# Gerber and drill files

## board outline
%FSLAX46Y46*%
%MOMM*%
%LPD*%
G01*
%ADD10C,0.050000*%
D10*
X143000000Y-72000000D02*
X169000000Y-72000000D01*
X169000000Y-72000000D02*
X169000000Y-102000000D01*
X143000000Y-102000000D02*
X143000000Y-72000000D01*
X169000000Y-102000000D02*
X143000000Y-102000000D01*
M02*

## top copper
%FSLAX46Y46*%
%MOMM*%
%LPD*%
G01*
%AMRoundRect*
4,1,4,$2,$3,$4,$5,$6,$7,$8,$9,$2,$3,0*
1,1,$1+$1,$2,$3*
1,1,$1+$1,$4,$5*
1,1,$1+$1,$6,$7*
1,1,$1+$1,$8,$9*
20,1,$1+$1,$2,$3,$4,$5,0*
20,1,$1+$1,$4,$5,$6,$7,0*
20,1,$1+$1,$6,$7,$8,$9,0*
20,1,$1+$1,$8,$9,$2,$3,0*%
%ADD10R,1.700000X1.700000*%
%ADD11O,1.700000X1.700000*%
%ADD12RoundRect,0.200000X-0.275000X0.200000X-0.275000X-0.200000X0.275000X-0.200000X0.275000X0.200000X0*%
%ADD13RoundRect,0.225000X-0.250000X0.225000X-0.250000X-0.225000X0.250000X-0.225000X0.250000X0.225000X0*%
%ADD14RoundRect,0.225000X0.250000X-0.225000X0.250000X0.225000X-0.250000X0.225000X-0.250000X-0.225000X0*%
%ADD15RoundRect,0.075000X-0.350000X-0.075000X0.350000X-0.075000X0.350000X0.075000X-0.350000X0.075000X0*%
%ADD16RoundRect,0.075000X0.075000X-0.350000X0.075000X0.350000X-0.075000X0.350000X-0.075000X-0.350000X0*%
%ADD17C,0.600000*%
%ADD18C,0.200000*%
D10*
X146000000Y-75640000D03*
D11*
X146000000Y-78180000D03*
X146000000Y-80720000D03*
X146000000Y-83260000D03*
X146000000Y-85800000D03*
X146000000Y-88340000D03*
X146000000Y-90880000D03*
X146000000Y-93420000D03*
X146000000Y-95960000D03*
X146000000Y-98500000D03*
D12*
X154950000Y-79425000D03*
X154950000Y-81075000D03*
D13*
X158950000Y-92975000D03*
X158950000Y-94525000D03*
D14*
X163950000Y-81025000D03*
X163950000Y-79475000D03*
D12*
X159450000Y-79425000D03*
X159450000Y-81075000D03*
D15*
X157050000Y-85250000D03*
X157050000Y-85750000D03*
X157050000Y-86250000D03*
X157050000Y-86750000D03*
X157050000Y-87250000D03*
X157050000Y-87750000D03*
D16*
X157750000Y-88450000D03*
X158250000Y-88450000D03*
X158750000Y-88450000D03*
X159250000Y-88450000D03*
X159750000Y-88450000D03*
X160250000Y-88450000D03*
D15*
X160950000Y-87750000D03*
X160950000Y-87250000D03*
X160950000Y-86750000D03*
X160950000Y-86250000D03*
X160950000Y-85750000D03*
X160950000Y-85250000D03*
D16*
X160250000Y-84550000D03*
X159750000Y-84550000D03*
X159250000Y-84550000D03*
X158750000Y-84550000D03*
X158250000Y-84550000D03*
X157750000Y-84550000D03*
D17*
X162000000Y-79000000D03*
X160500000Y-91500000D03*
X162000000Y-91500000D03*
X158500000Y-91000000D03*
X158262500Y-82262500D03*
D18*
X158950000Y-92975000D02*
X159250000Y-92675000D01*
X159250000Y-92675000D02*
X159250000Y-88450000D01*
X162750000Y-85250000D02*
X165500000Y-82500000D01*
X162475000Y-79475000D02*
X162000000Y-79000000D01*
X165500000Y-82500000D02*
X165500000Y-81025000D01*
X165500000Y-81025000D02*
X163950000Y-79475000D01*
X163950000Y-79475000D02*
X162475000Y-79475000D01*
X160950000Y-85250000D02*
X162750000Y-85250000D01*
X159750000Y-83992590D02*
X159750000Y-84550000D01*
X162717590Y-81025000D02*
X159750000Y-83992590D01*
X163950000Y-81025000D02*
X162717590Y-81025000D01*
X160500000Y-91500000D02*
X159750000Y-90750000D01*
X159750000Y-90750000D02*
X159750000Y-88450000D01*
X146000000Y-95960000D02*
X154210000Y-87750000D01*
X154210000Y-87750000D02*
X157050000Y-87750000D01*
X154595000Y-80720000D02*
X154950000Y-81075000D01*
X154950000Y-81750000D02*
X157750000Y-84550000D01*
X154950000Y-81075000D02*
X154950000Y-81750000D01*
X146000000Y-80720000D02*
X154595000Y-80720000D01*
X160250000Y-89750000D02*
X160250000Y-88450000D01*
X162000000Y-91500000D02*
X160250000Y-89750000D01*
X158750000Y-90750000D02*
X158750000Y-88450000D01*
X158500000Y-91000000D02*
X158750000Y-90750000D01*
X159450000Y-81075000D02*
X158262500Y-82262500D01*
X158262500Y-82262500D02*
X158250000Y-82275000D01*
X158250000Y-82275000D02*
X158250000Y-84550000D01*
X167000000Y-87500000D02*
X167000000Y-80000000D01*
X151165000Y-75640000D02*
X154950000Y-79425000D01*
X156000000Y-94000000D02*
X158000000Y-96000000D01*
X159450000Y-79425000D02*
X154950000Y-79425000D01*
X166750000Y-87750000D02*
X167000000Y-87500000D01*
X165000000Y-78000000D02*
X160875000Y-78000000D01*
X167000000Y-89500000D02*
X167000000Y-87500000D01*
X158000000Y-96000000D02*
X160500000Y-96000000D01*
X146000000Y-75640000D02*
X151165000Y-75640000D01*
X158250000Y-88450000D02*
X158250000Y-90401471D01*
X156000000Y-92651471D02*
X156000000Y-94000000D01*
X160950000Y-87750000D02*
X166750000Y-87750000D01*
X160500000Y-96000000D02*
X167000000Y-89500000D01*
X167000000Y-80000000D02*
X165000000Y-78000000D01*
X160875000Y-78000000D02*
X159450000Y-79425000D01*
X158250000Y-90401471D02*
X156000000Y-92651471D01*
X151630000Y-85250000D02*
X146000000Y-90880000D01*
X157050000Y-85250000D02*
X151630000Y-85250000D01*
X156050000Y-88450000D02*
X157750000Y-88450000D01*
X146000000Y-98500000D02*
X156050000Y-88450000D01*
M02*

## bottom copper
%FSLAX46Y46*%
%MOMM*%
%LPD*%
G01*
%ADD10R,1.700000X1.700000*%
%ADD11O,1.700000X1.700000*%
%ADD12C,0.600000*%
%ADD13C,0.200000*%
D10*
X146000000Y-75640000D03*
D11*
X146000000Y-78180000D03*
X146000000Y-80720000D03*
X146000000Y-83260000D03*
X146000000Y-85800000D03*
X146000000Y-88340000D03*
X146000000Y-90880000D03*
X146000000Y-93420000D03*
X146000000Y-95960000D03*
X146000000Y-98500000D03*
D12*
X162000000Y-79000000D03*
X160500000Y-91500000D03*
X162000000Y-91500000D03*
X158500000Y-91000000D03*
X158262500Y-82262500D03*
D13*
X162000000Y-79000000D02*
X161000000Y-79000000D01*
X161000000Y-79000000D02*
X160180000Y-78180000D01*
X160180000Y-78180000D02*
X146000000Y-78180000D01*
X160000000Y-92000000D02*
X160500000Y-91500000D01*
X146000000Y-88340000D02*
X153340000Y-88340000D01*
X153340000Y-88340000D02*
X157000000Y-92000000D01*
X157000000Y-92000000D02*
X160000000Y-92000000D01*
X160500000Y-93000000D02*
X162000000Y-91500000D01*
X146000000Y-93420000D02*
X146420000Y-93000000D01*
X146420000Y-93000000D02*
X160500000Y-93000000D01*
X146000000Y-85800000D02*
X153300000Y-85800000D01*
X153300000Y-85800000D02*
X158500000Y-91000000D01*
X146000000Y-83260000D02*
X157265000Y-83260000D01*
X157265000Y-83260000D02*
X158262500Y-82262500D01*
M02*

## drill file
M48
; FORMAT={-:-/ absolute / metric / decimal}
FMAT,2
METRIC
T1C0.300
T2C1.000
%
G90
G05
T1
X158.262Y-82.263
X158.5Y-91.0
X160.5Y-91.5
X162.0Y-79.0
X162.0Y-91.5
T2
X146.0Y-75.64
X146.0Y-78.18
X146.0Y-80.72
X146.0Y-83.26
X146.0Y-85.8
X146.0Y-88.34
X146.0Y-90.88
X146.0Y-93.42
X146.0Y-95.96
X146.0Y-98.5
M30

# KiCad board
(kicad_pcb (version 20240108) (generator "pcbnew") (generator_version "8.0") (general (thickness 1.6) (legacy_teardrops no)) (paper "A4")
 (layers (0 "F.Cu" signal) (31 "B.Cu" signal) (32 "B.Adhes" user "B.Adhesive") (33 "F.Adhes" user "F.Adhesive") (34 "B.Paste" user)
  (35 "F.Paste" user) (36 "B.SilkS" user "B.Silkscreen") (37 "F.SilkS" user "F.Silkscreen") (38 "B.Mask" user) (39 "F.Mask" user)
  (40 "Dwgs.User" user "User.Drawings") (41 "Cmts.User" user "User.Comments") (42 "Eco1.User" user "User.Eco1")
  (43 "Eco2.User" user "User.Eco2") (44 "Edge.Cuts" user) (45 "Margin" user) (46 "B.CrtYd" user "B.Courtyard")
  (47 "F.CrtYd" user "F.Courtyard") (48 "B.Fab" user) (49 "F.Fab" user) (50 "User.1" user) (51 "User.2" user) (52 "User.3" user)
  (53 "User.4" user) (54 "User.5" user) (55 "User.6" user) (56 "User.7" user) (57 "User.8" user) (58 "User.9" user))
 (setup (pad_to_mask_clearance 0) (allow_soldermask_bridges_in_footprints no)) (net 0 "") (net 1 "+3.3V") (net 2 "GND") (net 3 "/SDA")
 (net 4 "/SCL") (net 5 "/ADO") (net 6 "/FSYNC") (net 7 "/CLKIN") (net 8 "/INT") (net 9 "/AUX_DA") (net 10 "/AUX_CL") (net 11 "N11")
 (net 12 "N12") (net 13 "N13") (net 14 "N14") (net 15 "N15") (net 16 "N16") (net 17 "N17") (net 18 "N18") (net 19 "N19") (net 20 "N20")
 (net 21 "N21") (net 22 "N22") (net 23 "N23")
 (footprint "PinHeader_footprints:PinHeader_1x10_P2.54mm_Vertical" (layer "F.Cu") (at 146 75.64)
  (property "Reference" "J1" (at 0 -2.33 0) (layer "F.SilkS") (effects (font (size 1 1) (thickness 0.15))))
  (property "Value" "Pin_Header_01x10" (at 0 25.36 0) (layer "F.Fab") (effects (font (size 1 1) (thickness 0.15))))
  (pad "1" thru_hole rect (at 0 0) (size 1.7 1.7) (drill 1) (layers "*.Cu" "*.Mask") (remove_unused_layers no) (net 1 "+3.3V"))
  (pad "2" thru_hole oval (at 0 2.54) (size 1.7 1.7) (drill 1) (layers "*.Cu" "*.Mask") (remove_unused_layers no) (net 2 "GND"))
  (pad "3" thru_hole oval (at 0 5.08) (size 1.7 1.7) (drill 1) (layers "*.Cu" "*.Mask") (remove_unused_layers no) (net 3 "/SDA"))
  (pad "4" thru_hole oval (at 0 7.62) (size 1.7 1.7) (drill 1) (layers "*.Cu" "*.Mask") (remove_unused_layers no) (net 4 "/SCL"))
  (pad "5" thru_hole oval (at 0 10.16) (size 1.7 1.7) (drill 1) (layers "*.Cu" "*.Mask") (remove_unused_layers no) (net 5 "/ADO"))
  (pad "6" thru_hole oval (at 0 12.7) (size 1.7 1.7) (drill 1) (layers "*.Cu" "*.Mask") (remove_unused_layers no) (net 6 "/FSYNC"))
  (pad "7" thru_hole oval (at 0 15.24) (size 1.7 1.7) (drill 1) (layers "*.Cu" "*.Mask") (remove_unused_layers no) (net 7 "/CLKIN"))
  (pad "8" thru_hole oval (at 0 17.78) (size 1.7 1.7) (drill 1) (layers "*.Cu" "*.Mask") (remove_unused_layers no) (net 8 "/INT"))
  (pad "9" thru_hole oval (at 0 20.32) (size 1.7 1.7) (drill 1) (layers "*.Cu" "*.Mask") (remove_unused_layers no) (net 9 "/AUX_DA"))
  (pad "10" thru_hole oval (at 0 22.86) (size 1.7 1.7) (drill 1) (layers "*.Cu" "*.Mask") (remove_unused_layers no) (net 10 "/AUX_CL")))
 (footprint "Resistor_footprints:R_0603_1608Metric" (layer "F.Cu") (at 154.95 80.25 -90)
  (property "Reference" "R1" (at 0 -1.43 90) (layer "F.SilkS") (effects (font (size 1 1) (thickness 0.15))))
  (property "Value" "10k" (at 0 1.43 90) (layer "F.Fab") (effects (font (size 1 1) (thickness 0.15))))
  (pad "1" smd roundrect (at -0.825 0 270) (size 0.8 0.95) (layers "F.Cu" "F.Paste" "F.Mask") (roundrect_rratio 0.25) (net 1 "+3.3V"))
  (pad "2" smd roundrect (at 0.825 0 270) (size 0.8 0.95) (layers "F.Cu" "F.Paste" "F.Mask") (roundrect_rratio 0.25) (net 3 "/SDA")))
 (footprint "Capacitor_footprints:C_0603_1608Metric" (layer "F.Cu") (at 158.95 93.75 -90)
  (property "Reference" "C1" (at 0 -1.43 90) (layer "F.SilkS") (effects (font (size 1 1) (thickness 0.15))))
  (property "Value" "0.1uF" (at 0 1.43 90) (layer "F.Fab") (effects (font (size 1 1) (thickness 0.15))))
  (pad "1" smd roundrect (at -0.775 0 270) (size 0.9 0.95) (layers "F.Cu" "F.Paste" "F.Mask") (roundrect_rratio 0.25) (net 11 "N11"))
  (pad "2" smd roundrect (at 0.775 0 270) (size 0.9 0.95) (layers "F.Cu" "F.Paste" "F.Mask") (roundrect_rratio 0.25) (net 2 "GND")))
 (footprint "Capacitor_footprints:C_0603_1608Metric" (layer "F.Cu") (at 163.95 80.25 90)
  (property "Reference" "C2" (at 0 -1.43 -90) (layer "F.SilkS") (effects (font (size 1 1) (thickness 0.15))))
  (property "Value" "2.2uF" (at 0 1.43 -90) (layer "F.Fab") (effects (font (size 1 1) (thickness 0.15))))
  (pad "1" smd roundrect (at -0.775 0 90) (size 0.9 0.95) (layers "F.Cu" "F.Paste" "F.Mask") (roundrect_rratio 0.25) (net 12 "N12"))
  (pad "2" smd roundrect (at 0.775 0 90) (size 0.9 0.95) (layers "F.Cu" "F.Paste" "F.Mask") (roundrect_rratio 0.25) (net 2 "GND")))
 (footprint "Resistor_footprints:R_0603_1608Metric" (layer "F.Cu") (at 159.45 80.25 -90)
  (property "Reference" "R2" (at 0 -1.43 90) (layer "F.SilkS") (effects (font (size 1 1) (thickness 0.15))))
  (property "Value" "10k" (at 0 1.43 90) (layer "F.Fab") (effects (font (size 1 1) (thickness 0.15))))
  (pad "1" smd roundrect (at -0.825 0 270) (size 0.8 0.95) (layers "F.Cu" "F.Paste" "F.Mask") (roundrect_rratio 0.25) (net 1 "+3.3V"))
  (pad "2" smd roundrect (at 0.825 0 270) (size 0.8 0.95) (layers "F.Cu" "F.Paste" "F.Mask") (roundrect_rratio 0.25) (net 4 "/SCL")))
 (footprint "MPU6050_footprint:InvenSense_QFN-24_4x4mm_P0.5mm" (layer "F.Cu") (at 159 86.5)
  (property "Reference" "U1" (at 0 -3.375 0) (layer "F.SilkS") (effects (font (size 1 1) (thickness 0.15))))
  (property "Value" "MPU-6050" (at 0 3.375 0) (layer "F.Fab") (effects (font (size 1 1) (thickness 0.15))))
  (pad "1" smd roundrect (at -1.95 -1.25) (size 0.85 0.3) (layers "F.Cu" "F.Paste" "F.Mask") (roundrect_rratio 0.25) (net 7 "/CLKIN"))
  (pad "2" smd roundrect (at -1.95 -0.75) (size 0.85 0.3) (layers "F.Cu" "F.Paste" "F.Mask") (roundrect_rratio 0.25) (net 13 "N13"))
  (pad "3" smd roundrect (at -1.95 -0.25) (size 0.85 0.3) (layers "F.Cu" "F.Paste" "F.Mask") (roundrect_rratio 0.25) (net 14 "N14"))
  (pad "4" smd roundrect (at -1.95 0.25) (size 0.85 0.3) (layers "F.Cu" "F.Paste" "F.Mask") (roundrect_rratio 0.25) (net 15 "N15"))
  (pad "5" smd roundrect (at -1.95 0.75) (size 0.85 0.3) (layers "F.Cu" "F.Paste" "F.Mask") (roundrect_rratio 0.25) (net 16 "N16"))
  (pad "6" smd roundrect (at -1.95 1.25) (size 0.85 0.3) (layers "F.Cu" "F.Paste" "F.Mask") (roundrect_rratio 0.25) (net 9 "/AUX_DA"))
  (pad "7" smd roundrect (at -1.25 1.95 90) (size 0.85 0.3) (layers "F.Cu" "F.Paste" "F.Mask") (roundrect_rratio 0.25) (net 10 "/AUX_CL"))
  (pad "8" smd roundrect (at -0.75 1.95 90) (size 0.85 0.3) (layers "F.Cu" "F.Paste" "F.Mask") (roundrect_rratio 0.25) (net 1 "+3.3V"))
  (pad "9" smd roundrect (at -0.25 1.95 90) (size 0.85 0.3) (layers "F.Cu" "F.Paste" "F.Mask") (roundrect_rratio 0.25) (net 5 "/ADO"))
  (pad "10" smd roundrect (at 0.25 1.95 90) (size 0.85 0.3) (layers "F.Cu" "F.Paste" "F.Mask") (roundrect_rratio 0.25) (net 11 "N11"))
  (pad "11" smd roundrect (at 0.75 1.95 90) (size 0.85 0.3) (layers "F.Cu" "F.Paste" "F.Mask") (roundrect_rratio 0.25) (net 6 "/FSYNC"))
  (pad "12" smd roundrect (at 1.25 1.95 90) (size 0.85 0.3) (layers "F.Cu" "F.Paste" "F.Mask") (roundrect_rratio 0.25) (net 8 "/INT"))
  (pad "13" smd roundrect (at 1.95 1.25) (size 0.85 0.3) (layers "F.Cu" "F.Paste" "F.Mask") (roundrect_rratio 0.25) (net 1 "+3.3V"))
  (pad "14" smd roundrect (at 1.95 0.75) (size 0.85 0.3) (layers "F.Cu" "F.Paste" "F.Mask") (roundrect_rratio 0.25) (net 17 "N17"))
  (pad "15" smd roundrect (at 1.95 0.25) (size 0.85 0.3) (layers "F.Cu" "F.Paste" "F.Mask") (roundrect_rratio 0.25) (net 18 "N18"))
  (pad "16" smd roundrect (at 1.95 -0.25) (size 0.85 0.3) (layers "F.Cu" "F.Paste" "F.Mask") (roundrect_rratio 0.25) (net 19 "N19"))
  (pad "17" smd roundrect (at 1.95 -0.75) (size 0.85 0.3) (layers "F.Cu" "F.Paste" "F.Mask") (roundrect_rratio 0.25) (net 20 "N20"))
  (pad "18" smd roundrect (at 1.95 -1.25) (size 0.85 0.3) (layers "F.Cu" "F.Paste" "F.Mask") (roundrect_rratio 0.25) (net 2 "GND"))
  (pad "19" smd roundrect (at 1.25 -1.95 90) (size 0.85 0.3) (layers "F.Cu" "F.Paste" "F.Mask") (roundrect_rratio 0.25) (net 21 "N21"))
  (pad "20" smd roundrect (at 0.75 -1.95 90) (size 0.85 0.3) (layers "F.Cu" "F.Paste" "F.Mask") (roundrect_rratio 0.25) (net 12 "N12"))
  (pad "21" smd roundrect (at 0.25 -1.95 90) (size 0.85 0.3) (layers "F.Cu" "F.Paste" "F.Mask") (roundrect_rratio 0.25) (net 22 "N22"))
  (pad "22" smd roundrect (at -0.25 -1.95 90) (size 0.85 0.3) (layers "F.Cu" "F.Paste" "F.Mask") (roundrect_rratio 0.25) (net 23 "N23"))
  (pad "23" smd roundrect (at -0.75 -1.95 90) (size 0.85 0.3) (layers "F.Cu" "F.Paste" "F.Mask") (roundrect_rratio 0.25) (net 4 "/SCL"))
  (pad "24" smd roundrect (at -1.25 -1.95 90) (size 0.85 0.3) (layers "F.Cu" "F.Paste" "F.Mask") (roundrect_rratio 0.25) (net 3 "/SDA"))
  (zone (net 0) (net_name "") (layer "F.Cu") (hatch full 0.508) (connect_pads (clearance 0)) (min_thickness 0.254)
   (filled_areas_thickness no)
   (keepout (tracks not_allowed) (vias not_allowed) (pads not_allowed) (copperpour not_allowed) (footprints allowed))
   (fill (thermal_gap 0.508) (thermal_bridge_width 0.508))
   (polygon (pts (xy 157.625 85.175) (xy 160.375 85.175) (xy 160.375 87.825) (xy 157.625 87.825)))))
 (gr_line (start 143 72) (end 169 72) (stroke (width 0.05) (type default)) (layer "Edge.Cuts"))
 (gr_line (start 169 72) (end 169 102) (stroke (width 0.05) (type default)) (layer "Edge.Cuts"))
 (gr_line (start 143 102) (end 143 72) (stroke (width 0.05) (type default)) (layer "Edge.Cuts"))
 (gr_line (start 169 102) (end 143 102) (stroke (width 0.05) (type default)) (layer "Edge.Cuts"))
 (segment (start 158.95 92.975) (end 159.25 92.675) (width 0.2) (layer "F.Cu") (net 11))
 (segment (start 159.25 92.675) (end 159.25 88.45) (width 0.2) (layer "F.Cu") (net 11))
 (segment (start 162.75 85.25) (end 165.5 82.5) (width 0.2) (layer "F.Cu") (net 2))
 (segment (start 162.475 79.475) (end 162 79) (width 0.2) (layer "F.Cu") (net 2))
 (segment (start 165.5 82.5) (end 165.5 81.025) (width 0.2) (layer "F.Cu") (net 2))
 (segment (start 165.5 81.025) (end 163.95 79.475) (width 0.2) (layer "F.Cu") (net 2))
 (segment (start 163.95 79.475) (end 162.475 79.475) (width 0.2) (layer "F.Cu") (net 2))
 (segment (start 160.95 85.25) (end 162.75 85.25) (width 0.2) (layer "F.Cu") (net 2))
 (via (at 162 79) (size 0.6) (drill 0.3) (layers "F.Cu" "B.Cu") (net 2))
 (segment (start 162 79) (end 161 79) (width 0.2) (layer "B.Cu") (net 2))
 (segment (start 161 79) (end 160.18 78.18) (width 0.2) (layer "B.Cu") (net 2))
 (segment (start 160.18 78.18) (end 146 78.18) (width 0.2) (layer "B.Cu") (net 2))
 (segment (start 159.75 83.99259) (end 159.75 84.55) (width 0.2) (layer "F.Cu") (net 12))
 (segment (start 162.71759 81.025) (end 159.75 83.99259) (width 0.2) (layer "F.Cu") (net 12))
 (segment (start 163.95 81.025) (end 162.71759 81.025) (width 0.2) (layer "F.Cu") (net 12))
 (segment (start 160.5 91.5) (end 159.75 90.75) (width 0.2) (layer "F.Cu") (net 6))
 (segment (start 159.75 90.75) (end 159.75 88.45) (width 0.2) (layer "F.Cu") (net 6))
 (via (at 160.5 91.5) (size 0.6) (drill 0.3) (layers "F.Cu" "B.Cu") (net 6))
 (segment (start 160 92) (end 160.5 91.5) (width 0.2) (layer "B.Cu") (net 6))
 (segment (start 146 88.34) (end 153.34 88.34) (width 0.2) (layer "B.Cu") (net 6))
 (segment (start 153.34 88.34) (end 157 92) (width 0.2) (layer "B.Cu") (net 6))
 (segment (start 157 92) (end 160 92) (width 0.2) (layer "B.Cu") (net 6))
 (segment (start 146 95.96) (end 154.21 87.75) (width 0.2) (layer "F.Cu") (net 9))
 (segment (start 154.21 87.75) (end 157.05 87.75) (width 0.2) (layer "F.Cu") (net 9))
 (segment (start 154.595 80.72) (end 154.95 81.075) (width 0.2) (layer "F.Cu") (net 3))
 (segment (start 154.95 81.75) (end 157.75 84.55) (width 0.2) (layer "F.Cu") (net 3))
 (segment (start 154.95 81.075) (end 154.95 81.75) (width 0.2) (layer "F.Cu") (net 3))
 (segment (start 146 80.72) (end 154.595 80.72) (width 0.2) (layer "F.Cu") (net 3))
 (segment (start 160.25 89.75) (end 160.25 88.45) (width 0.2) (layer "F.Cu") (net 8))
 (segment (start 162 91.5) (end 160.25 89.75) (width 0.2) (layer "F.Cu") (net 8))
 (via (at 162 91.5) (size 0.6) (drill 0.3) (layers "F.Cu" "B.Cu") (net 8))
 (segment (start 160.5 93) (end 162 91.5) (width 0.2) (layer "B.Cu") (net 8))
 (segment (start 146 93.42) (end 146.42 93) (width 0.2) (layer "B.Cu") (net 8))
 (segment (start 146.42 93) (end 160.5 93) (width 0.2) (layer "B.Cu") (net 8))
 (segment (start 158.75 90.75) (end 158.75 88.45) (width 0.2) (layer "F.Cu") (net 5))
 (segment (start 158.5 91) (end 158.75 90.75) (width 0.2) (layer "F.Cu") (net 5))
 (via (at 158.5 91) (size 0.6) (drill 0.3) (layers "F.Cu" "B.Cu") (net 5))
 (segment (start 146 85.8) (end 153.3 85.8) (width 0.2) (layer "B.Cu") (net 5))
 (segment (start 153.3 85.8) (end 158.5 91) (width 0.2) (layer "B.Cu") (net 5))
 (segment (start 159.45 81.075) (end 158.2625 82.2625) (width 0.2) (layer "F.Cu") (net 4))
 (segment (start 158.2625 82.2625) (end 158.25 82.275) (width 0.2) (layer "F.Cu") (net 4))
 (segment (start 158.25 82.275) (end 158.25 84.55) (width 0.2) (layer "F.Cu") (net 4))
 (via (at 158.2625 82.2625) (size 0.6) (drill 0.3) (layers "F.Cu" "B.Cu") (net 4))
 (segment (start 146 83.26) (end 157.265 83.26) (width 0.2) (layer "B.Cu") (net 4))
 (segment (start 157.265 83.26) (end 158.2625 82.2625) (width 0.2) (layer "B.Cu") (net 4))
 (segment (start 167 87.5) (end 167 80) (width 0.2) (layer "F.Cu") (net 1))
 (segment (start 151.165 75.64) (end 154.95 79.425) (width 0.2) (layer "F.Cu") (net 1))
 (segment (start 156 94) (end 158 96) (width 0.2) (layer "F.Cu") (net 1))
 (segment (start 159.45 79.425) (end 154.95 79.425) (width 0.2) (layer "F.Cu") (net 1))
 (segment (start 166.75 87.75) (end 167 87.5) (width 0.2) (layer "F.Cu") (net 1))
 (segment (start 165 78) (end 160.875 78) (width 0.2) (layer "F.Cu") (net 1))
 (segment (start 167 89.5) (end 167 87.5) (width 0.2) (layer "F.Cu") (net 1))
 (segment (start 158 96) (end 160.5 96) (width 0.2) (layer "F.Cu") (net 1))
 (segment (start 146 75.64) (end 151.165 75.64) (width 0.2) (layer "F.Cu") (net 1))
 (segment (start 158.25 88.45) (end 158.25 90.401471) (width 0.2) (layer "F.Cu") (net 1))
 (segment (start 156 92.651471) (end 156 94) (width 0.2) (layer "F.Cu") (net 1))
 (segment (start 160.95 87.75) (end 166.75 87.75) (width 0.2) (layer "F.Cu") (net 1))
 (segment (start 160.5 96) (end 167 89.5) (width 0.2) (layer "F.Cu") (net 1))
 (segment (start 167 80) (end 165 78) (width 0.2) (layer "F.Cu") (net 1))
 (segment (start 160.875 78) (end 159.45 79.425) (width 0.2) (layer "F.Cu") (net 1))
 (segment (start 158.25 90.401471) (end 156 92.651471) (width 0.2) (layer "F.Cu") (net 1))
 (segment (start 151.63 85.25) (end 146 90.88) (width 0.2) (layer "F.Cu") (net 7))
 (segment (start 157.05 85.25) (end 151.63 85.25) (width 0.2) (layer "F.Cu") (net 7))
 (segment (start 156.05 88.45) (end 157.75 88.45) (width 0.2) (layer "F.Cu") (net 10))
 (segment (start 146 98.5) (end 156.05 88.45) (width 0.2) (layer "F.Cu") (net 10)))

